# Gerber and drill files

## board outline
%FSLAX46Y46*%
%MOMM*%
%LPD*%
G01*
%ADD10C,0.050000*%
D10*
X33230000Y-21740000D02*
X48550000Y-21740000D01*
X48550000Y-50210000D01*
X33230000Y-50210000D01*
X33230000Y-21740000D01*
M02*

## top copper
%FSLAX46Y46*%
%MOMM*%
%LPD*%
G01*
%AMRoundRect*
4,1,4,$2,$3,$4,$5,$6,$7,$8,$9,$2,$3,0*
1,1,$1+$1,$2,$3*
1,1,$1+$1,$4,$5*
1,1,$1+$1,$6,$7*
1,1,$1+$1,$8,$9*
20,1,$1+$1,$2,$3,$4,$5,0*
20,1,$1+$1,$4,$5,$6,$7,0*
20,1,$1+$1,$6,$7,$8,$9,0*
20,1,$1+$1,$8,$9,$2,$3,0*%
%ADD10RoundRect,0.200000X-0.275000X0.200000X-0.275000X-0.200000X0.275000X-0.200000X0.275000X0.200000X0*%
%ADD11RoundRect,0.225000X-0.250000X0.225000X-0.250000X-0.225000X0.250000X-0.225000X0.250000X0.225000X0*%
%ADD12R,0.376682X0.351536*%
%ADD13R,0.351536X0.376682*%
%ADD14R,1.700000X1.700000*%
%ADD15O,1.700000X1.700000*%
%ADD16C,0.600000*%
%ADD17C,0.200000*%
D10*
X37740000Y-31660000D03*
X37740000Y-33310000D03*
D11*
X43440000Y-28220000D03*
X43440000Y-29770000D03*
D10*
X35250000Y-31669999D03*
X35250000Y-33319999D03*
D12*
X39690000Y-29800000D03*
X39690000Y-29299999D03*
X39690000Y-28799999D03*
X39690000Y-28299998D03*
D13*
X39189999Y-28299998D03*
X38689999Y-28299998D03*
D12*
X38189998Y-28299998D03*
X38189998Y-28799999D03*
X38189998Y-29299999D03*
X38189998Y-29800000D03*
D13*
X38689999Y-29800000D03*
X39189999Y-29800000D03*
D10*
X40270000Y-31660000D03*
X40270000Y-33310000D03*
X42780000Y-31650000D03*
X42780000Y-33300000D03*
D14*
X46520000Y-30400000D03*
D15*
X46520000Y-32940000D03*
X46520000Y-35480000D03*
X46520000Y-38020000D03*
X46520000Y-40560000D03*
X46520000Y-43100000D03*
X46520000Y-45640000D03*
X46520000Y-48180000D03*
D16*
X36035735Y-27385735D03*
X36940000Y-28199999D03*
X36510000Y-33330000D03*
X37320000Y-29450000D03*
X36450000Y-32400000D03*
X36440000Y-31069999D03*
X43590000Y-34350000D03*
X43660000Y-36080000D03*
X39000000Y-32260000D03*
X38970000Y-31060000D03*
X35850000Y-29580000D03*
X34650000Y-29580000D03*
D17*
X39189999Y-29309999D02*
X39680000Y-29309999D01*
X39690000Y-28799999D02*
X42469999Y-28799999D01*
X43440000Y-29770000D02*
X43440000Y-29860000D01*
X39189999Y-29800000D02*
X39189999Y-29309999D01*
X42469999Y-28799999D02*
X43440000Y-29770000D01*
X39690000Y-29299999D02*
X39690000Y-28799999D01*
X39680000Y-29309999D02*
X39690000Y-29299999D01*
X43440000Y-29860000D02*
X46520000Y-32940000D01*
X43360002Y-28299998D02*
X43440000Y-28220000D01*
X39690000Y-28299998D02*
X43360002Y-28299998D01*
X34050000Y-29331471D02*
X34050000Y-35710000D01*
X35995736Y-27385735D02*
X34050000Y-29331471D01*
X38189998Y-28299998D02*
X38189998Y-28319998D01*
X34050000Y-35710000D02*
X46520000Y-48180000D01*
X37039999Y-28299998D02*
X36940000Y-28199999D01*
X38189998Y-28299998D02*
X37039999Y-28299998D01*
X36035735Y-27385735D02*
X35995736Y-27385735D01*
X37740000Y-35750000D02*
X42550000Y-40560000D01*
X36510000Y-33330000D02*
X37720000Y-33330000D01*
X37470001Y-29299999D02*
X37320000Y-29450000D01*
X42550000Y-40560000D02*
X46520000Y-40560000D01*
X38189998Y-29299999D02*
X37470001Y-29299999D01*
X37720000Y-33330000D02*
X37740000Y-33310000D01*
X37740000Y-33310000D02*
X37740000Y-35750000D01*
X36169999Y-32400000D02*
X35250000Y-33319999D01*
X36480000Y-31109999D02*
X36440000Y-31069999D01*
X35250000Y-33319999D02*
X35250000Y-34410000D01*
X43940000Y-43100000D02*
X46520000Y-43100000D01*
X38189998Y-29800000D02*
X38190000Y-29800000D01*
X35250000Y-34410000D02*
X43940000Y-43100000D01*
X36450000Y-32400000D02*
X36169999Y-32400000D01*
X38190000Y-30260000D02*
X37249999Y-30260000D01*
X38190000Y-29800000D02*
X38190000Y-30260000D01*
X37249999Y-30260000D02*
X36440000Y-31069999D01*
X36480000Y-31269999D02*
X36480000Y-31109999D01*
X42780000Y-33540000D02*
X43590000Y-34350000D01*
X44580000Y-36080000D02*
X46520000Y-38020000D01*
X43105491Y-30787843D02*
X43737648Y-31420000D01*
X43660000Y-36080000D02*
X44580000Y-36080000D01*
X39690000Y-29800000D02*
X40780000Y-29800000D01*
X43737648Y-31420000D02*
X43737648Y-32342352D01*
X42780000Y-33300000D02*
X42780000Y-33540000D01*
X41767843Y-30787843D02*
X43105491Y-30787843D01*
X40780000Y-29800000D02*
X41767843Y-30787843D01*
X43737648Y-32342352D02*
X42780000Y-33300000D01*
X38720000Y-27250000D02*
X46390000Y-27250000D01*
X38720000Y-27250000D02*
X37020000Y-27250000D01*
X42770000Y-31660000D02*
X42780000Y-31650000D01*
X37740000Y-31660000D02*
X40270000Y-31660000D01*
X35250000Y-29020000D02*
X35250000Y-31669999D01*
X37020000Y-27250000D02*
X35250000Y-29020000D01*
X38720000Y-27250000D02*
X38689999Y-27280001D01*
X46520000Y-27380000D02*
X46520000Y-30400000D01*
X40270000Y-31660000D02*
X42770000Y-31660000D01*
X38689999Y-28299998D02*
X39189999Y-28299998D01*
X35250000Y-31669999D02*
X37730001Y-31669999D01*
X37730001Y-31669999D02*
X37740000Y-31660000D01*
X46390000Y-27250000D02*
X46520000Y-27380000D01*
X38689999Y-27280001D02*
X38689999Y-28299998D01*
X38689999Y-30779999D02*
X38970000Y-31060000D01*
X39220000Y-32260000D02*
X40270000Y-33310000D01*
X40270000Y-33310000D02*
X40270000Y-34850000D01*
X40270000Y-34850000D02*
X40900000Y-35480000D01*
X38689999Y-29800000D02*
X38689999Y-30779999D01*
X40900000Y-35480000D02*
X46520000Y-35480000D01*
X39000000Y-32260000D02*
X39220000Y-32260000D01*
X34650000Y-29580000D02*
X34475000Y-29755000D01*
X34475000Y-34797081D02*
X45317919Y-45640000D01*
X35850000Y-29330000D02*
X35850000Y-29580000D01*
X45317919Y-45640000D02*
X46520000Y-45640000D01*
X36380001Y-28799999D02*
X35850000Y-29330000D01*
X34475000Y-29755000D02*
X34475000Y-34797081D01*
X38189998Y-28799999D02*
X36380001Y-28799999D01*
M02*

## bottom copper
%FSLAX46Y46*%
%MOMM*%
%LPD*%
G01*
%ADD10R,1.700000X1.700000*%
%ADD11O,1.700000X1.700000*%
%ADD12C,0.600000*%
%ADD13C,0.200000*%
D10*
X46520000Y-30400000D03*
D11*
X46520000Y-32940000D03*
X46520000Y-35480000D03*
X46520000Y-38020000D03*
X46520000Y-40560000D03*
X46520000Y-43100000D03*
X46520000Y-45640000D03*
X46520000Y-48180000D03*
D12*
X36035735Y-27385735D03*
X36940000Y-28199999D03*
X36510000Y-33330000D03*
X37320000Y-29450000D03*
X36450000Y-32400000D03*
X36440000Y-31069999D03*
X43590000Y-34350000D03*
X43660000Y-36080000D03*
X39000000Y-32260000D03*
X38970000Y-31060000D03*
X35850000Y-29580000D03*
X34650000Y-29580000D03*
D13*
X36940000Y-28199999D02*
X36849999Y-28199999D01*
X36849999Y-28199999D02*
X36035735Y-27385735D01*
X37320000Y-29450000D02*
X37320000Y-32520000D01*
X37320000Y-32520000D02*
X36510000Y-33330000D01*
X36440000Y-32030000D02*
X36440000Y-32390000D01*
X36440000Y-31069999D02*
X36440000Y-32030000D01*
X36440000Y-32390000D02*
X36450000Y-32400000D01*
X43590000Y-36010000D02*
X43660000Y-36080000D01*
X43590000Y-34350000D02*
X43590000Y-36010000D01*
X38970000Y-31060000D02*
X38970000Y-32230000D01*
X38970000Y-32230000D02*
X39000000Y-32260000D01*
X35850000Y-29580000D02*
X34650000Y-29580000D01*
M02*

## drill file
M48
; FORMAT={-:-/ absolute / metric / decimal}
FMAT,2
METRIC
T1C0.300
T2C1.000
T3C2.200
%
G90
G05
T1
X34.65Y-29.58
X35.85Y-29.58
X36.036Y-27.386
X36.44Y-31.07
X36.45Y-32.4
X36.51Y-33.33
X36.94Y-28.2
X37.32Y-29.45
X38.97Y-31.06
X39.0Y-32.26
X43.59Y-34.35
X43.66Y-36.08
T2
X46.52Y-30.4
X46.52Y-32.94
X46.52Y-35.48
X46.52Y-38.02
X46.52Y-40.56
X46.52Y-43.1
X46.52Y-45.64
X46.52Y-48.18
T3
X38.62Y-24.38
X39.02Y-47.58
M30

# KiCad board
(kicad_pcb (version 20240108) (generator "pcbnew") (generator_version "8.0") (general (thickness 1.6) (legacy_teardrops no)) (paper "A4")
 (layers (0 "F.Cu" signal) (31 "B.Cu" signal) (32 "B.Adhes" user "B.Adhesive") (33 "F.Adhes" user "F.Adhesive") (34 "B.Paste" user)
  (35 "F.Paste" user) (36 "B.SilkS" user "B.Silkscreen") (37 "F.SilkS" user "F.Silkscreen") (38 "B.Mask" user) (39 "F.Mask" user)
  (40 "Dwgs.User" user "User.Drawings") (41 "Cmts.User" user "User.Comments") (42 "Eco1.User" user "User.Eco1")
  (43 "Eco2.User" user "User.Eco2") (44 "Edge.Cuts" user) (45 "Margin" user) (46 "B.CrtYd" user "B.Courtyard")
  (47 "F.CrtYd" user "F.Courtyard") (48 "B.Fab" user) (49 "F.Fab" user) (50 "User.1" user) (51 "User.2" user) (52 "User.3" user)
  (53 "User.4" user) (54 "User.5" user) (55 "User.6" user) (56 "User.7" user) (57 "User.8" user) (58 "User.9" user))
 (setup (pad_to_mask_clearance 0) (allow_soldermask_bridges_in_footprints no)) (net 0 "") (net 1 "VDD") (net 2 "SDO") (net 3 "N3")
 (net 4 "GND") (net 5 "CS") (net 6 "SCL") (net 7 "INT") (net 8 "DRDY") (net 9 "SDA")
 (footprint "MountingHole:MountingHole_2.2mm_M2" (layer "F.Cu") (at 39.02 47.58)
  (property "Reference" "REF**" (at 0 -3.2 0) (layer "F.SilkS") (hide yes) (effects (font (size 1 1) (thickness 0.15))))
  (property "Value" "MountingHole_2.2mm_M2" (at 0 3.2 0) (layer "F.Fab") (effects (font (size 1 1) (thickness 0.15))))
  (pad "" np_thru_hole circle (at 0 0) (size 2.2 2.2) (drill 2.2) (layers "*.Cu" "*.Mask")))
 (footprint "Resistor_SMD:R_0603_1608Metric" (layer "F.Cu") (at 37.74 32.485 -90)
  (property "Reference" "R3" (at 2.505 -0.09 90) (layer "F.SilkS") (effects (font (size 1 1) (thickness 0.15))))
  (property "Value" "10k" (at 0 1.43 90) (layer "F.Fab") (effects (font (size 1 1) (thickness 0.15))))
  (pad "1" smd roundrect (at -0.825 0 270) (size 0.8 0.95) (layers "F.Cu" "F.Paste" "F.Mask") (roundrect_rratio 0.25) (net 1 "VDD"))
  (pad "2" smd roundrect (at 0.825 0 270) (size 0.8 0.95) (layers "F.Cu" "F.Paste" "F.Mask") (roundrect_rratio 0.25) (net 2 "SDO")))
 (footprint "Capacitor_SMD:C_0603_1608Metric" (layer "F.Cu") (at 43.44 28.995 -90)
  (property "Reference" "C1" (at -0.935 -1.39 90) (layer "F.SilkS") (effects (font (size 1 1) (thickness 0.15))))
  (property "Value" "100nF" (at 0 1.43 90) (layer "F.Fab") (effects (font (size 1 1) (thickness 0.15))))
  (pad "1" smd roundrect (at -0.775 0 270) (size 0.9 0.95) (layers "F.Cu" "F.Paste" "F.Mask") (roundrect_rratio 0.25) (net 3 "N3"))
  (pad "2" smd roundrect (at 0.775 0 270) (size 0.9 0.95) (layers "F.Cu" "F.Paste" "F.Mask") (roundrect_rratio 0.25) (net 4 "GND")))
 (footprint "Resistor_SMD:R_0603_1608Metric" (layer "F.Cu") (at 35.25 32.494999 -90)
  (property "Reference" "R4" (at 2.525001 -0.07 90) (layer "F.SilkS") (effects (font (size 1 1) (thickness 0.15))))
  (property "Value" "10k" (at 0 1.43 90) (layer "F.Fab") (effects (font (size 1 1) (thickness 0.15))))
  (pad "1" smd roundrect (at -0.825 0 270) (size 0.8 0.95) (layers "F.Cu" "F.Paste" "F.Mask") (roundrect_rratio 0.25) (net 1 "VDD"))
  (pad "2" smd roundrect (at 0.825 0 270) (size 0.8 0.95) (layers "F.Cu" "F.Paste" "F.Mask") (roundrect_rratio 0.25) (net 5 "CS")))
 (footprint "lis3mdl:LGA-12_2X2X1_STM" (layer "F.Cu") (at 38.939999 29.049999 180)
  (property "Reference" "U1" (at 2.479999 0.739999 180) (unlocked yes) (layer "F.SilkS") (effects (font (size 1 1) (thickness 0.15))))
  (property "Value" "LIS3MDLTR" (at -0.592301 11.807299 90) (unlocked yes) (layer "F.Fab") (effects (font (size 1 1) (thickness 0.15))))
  (pad "1" smd rect (at -0.750001 -0.750001 180) (size 0.376682 0.351536) (layers "F.Cu" "F.Paste" "F.Mask") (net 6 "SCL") (clearance 0.05))
  (pad "2" smd rect (at -0.750001 -0.25 180) (size 0.376682 0.351536) (layers "F.Cu" "F.Paste" "F.Mask") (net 4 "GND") (clearance 0.05))
  (pad "3" smd rect (at -0.750001 0.25 180) (size 0.376682 0.351536) (layers "F.Cu" "F.Paste" "F.Mask") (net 4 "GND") (clearance 0.05))
  (pad "4" smd rect (at -0.750001 0.750001 180) (size 0.376682 0.351536) (layers "F.Cu" "F.Paste" "F.Mask") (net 3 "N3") (clearance 0.05))
  (pad "5" smd rect (at -0.25 0.750001 270) (size 0.376682 0.351536) (layers "F.Cu" "F.Paste" "F.Mask") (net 1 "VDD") (clearance 0.05))
  (pad "6" smd rect (at 0.25 0.750001 270) (size 0.376682 0.351536) (layers "F.Cu" "F.Paste" "F.Mask") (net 1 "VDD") (clearance 0.05))
  (pad "7" smd rect (at 0.750001 0.750001 180) (size 0.376682 0.351536) (layers "F.Cu" "F.Paste" "F.Mask") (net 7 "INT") (clearance 0.05))
  (pad "8" smd rect (at 0.750001 0.25 180) (size 0.376682 0.351536) (layers "F.Cu" "F.Paste" "F.Mask") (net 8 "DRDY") (clearance 0.05))
  (pad "9" smd rect (at 0.750001 -0.25 180) (size 0.376682 0.351536) (layers "F.Cu" "F.Paste" "F.Mask") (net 2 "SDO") (clearance 0.05))
  (pad "10" smd rect (at 0.750001 -0.750001 180) (size 0.376682 0.351536) (layers "F.Cu" "F.Paste" "F.Mask") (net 5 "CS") (clearance 0.05))
  (pad "11" smd rect (at 0.25 -0.750001 270) (size 0.376682 0.351536) (layers "F.Cu" "F.Paste" "F.Mask") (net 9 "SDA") (clearance 0.05))
  (pad "12" smd rect (at -0.25 -0.750001 270) (size 0.376682 0.351536) (layers "F.Cu" "F.Paste" "F.Mask") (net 4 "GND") (clearance 0.05)))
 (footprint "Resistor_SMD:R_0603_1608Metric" (layer "F.Cu") (at 40.27 32.485 -90)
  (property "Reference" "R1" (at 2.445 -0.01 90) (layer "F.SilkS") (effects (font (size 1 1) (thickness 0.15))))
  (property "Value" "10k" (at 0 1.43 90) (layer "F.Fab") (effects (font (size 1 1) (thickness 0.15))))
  (pad "1" smd roundrect (at -0.825 0 270) (size 0.8 0.95) (layers "F.Cu" "F.Paste" "F.Mask") (roundrect_rratio 0.25) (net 1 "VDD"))
  (pad "2" smd roundrect (at 0.825 0 270) (size 0.8 0.95) (layers "F.Cu" "F.Paste" "F.Mask") (roundrect_rratio 0.25) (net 9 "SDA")))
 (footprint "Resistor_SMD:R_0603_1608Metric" (layer "F.Cu") (at 42.78 32.475 -90)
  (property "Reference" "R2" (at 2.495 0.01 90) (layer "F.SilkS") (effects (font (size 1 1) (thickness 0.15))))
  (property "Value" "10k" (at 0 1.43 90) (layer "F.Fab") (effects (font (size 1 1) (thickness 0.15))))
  (pad "1" smd roundrect (at -0.825 0 270) (size 0.8 0.95) (layers "F.Cu" "F.Paste" "F.Mask") (roundrect_rratio 0.25) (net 1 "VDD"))
  (pad "2" smd roundrect (at 0.825 0 270) (size 0.8 0.95) (layers "F.Cu" "F.Paste" "F.Mask") (roundrect_rratio 0.25) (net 6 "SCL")))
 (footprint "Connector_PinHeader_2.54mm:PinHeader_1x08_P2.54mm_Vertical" (layer "F.Cu") (at 46.52 30.4)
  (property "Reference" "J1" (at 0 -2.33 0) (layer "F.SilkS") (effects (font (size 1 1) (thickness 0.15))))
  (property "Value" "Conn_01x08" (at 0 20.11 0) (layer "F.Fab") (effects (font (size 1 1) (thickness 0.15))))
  (pad "1" thru_hole rect (at 0 0) (size 1.7 1.7) (drill 1) (layers "*.Cu" "*.Mask") (remove_unused_layers no) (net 1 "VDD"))
  (pad "2" thru_hole oval (at 0 2.54) (size 1.7 1.7) (drill 1) (layers "*.Cu" "*.Mask") (remove_unused_layers no) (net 4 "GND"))
  (pad "3" thru_hole oval (at 0 5.08) (size 1.7 1.7) (drill 1) (layers "*.Cu" "*.Mask") (remove_unused_layers no) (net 9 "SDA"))
  (pad "4" thru_hole oval (at 0 7.62) (size 1.7 1.7) (drill 1) (layers "*.Cu" "*.Mask") (remove_unused_layers no) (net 6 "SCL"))
  (pad "5" thru_hole oval (at 0 10.16) (size 1.7 1.7) (drill 1) (layers "*.Cu" "*.Mask") (remove_unused_layers no) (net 2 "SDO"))
  (pad "6" thru_hole oval (at 0 12.7) (size 1.7 1.7) (drill 1) (layers "*.Cu" "*.Mask") (remove_unused_layers no) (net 5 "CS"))
  (pad "7" thru_hole oval (at 0 15.24) (size 1.7 1.7) (drill 1) (layers "*.Cu" "*.Mask") (remove_unused_layers no) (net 8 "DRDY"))
  (pad "8" thru_hole oval (at 0 17.78) (size 1.7 1.7) (drill 1) (layers "*.Cu" "*.Mask") (remove_unused_layers no) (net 7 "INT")))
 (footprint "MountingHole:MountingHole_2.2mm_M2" (layer "F.Cu") (at 38.62 24.38)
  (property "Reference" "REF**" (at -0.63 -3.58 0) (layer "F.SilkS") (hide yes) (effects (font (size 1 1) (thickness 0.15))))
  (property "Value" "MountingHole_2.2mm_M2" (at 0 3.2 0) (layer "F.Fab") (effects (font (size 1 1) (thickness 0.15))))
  (pad "" np_thru_hole circle (at 0 0) (size 2.2 2.2) (drill 2.2) (layers "*.Cu" "*.Mask")))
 (gr_rect (start 33.23 21.74) (end 48.55 50.21) (stroke (width 0.05) (type default)) (fill none) (layer "Edge.Cuts"))
 (segment (start 39.189999 29.309999) (end 39.68 29.309999) (width 0.2) (layer "F.Cu") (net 4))
 (segment (start 39.69 28.799999) (end 42.469999 28.799999) (width 0.2) (layer "F.Cu") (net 4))
 (segment (start 43.44 29.77) (end 43.44 29.86) (width 0.2) (layer "F.Cu") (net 4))
 (segment (start 39.189999 29.8) (end 39.189999 29.309999) (width 0.2) (layer "F.Cu") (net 4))
 (segment (start 42.469999 28.799999) (end 43.44 29.77) (width 0.2) (layer "F.Cu") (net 4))
 (segment (start 39.69 29.299999) (end 39.69 28.799999) (width 0.2) (layer "F.Cu") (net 4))
 (segment (start 39.68 29.309999) (end 39.69 29.299999) (width 0.2) (layer "F.Cu") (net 4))
 (segment (start 43.44 29.86) (end 46.52 32.94) (width 0.2) (layer "F.Cu") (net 4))
 (segment (start 43.360002 28.299998) (end 43.44 28.22) (width 0.2) (layer "F.Cu") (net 3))
 (segment (start 39.69 28.299998) (end 43.360002 28.299998) (width 0.2) (layer "F.Cu") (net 3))
 (segment (start 34.05 29.331471) (end 34.05 35.71) (width 0.2) (layer "F.Cu") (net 7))
 (segment (start 35.995736 27.385735) (end 34.05 29.331471) (width 0.2) (layer "F.Cu") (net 7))
 (segment (start 38.189998 28.299998) (end 38.189998 28.319998) (width 0.2) (layer "F.Cu") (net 7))
 (segment (start 34.05 35.71) (end 46.52 48.18) (width 0.2) (layer "F.Cu") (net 7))
 (segment (start 37.039999 28.299998) (end 36.94 28.199999) (width 0.2) (layer "F.Cu") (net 7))
 (segment (start 38.189998 28.299998) (end 37.039999 28.299998) (width 0.2) (layer "F.Cu") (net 7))
 (segment (start 36.035735 27.385735) (end 35.995736 27.385735) (width 0.2) (layer "F.Cu") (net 7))
 (via (at 36.035735 27.385735) (size 0.6) (drill 0.3) (layers "F.Cu" "B.Cu") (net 7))
 (via (at 36.94 28.199999) (size 0.6) (drill 0.3) (layers "F.Cu" "B.Cu") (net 7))
 (segment (start 36.94 28.199999) (end 36.849999 28.199999) (width 0.2) (layer "B.Cu") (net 7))
 (segment (start 36.849999 28.199999) (end 36.035735 27.385735) (width 0.2) (layer "B.Cu") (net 7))
 (segment (start 37.74 35.75) (end 42.55 40.56) (width 0.2) (layer "F.Cu") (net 2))
 (segment (start 36.51 33.33) (end 37.72 33.33) (width 0.2) (layer "F.Cu") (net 2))
 (segment (start 37.470001 29.299999) (end 37.32 29.45) (width 0.2) (layer "F.Cu") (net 2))
 (segment (start 42.55 40.56) (end 46.52 40.56) (width 0.2) (layer "F.Cu") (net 2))
 (segment (start 38.189998 29.299999) (end 37.470001 29.299999) (width 0.2) (layer "F.Cu") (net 2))
 (segment (start 37.72 33.33) (end 37.74 33.31) (width 0.2) (layer "F.Cu") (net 2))
 (segment (start 37.74 33.31) (end 37.74 35.75) (width 0.2) (layer "F.Cu") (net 2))
 (via (at 36.51 33.33) (size 0.6) (drill 0.3) (layers "F.Cu" "B.Cu") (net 2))
 (via (at 37.32 29.45) (size 0.6) (drill 0.3) (layers "F.Cu" "B.Cu") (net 2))
 (segment (start 37.32 29.45) (end 37.32 32.52) (width 0.2) (layer "B.Cu") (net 2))
 (segment (start 37.32 32.52) (end 36.51 33.33) (width 0.2) (layer "B.Cu") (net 2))
 (segment (start 36.169999 32.4) (end 35.25 33.319999) (width 0.2) (layer "F.Cu") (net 5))
 (segment (start 36.48 31.109999) (end 36.44 31.069999) (width 0.2) (layer "F.Cu") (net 5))
 (segment (start 35.25 33.319999) (end 35.25 34.41) (width 0.2) (layer "F.Cu") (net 5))
 (segment (start 43.94 43.1) (end 46.52 43.1) (width 0.2) (layer "F.Cu") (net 5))
 (segment (start 38.189998 29.8) (end 38.19 29.8) (width 0.2) (layer "F.Cu") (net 5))
 (segment (start 35.25 34.41) (end 43.94 43.1) (width 0.2) (layer "F.Cu") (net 5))
 (segment (start 36.45 32.4) (end 36.169999 32.4) (width 0.2) (layer "F.Cu") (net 5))
 (segment (start 38.19 30.26) (end 37.249999 30.26) (width 0.2) (layer "F.Cu") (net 5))
 (segment (start 38.19 29.8) (end 38.19 30.26) (width 0.2) (layer "F.Cu") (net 5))
 (segment (start 37.249999 30.26) (end 36.44 31.069999) (width 0.2) (layer "F.Cu") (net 5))
 (segment (start 36.48 31.269999) (end 36.48 31.109999) (width 0.2) (layer "F.Cu") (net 5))
 (via (at 36.45 32.4) (size 0.6) (drill 0.3) (layers "F.Cu" "B.Cu") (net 5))
 (via (at 36.44 31.069999) (size 0.6) (drill 0.3) (layers "F.Cu" "B.Cu") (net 5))
 (segment (start 36.44 32.03) (end 36.44 32.39) (width 0.2) (layer "B.Cu") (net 5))
 (segment (start 36.44 31.069999) (end 36.44 32.03) (width 0.2) (layer "B.Cu") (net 5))
 (segment (start 36.44 32.39) (end 36.45 32.4) (width 0.2) (layer "B.Cu") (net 5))
 (segment (start 42.78 33.54) (end 43.59 34.35) (width 0.2) (layer "F.Cu") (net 6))
 (segment (start 44.58 36.08) (end 46.52 38.02) (width 0.2) (layer "F.Cu") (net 6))
 (segment (start 43.105491 30.787843) (end 43.737648 31.42) (width 0.2) (layer "F.Cu") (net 6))
 (segment (start 43.66 36.08) (end 44.58 36.08) (width 0.2) (layer "F.Cu") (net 6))
 (segment (start 39.69 29.8) (end 40.78 29.8) (width 0.2) (layer "F.Cu") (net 6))
 (segment (start 43.737648 31.42) (end 43.737648 32.342352) (width 0.2) (layer "F.Cu") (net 6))
 (segment (start 42.78 33.3) (end 42.78 33.54) (width 0.2) (layer "F.Cu") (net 6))
 (segment (start 41.767843 30.787843) (end 43.105491 30.787843) (width 0.2) (layer "F.Cu") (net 6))
 (segment (start 40.78 29.8) (end 41.767843 30.787843) (width 0.2) (layer "F.Cu") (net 6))
 (segment (start 43.737648 32.342352) (end 42.78 33.3) (width 0.2) (layer "F.Cu") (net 6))
 (via (at 43.59 34.35) (size 0.6) (drill 0.3) (layers "F.Cu" "B.Cu") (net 6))
 (via (at 43.66 36.08) (size 0.6) (drill 0.3) (layers "F.Cu" "B.Cu") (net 6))
 (segment (start 43.59 36.01) (end 43.66 36.08) (width 0.2) (layer "B.Cu") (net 6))
 (segment (start 43.59 34.35) (end 43.59 36.01) (width 0.2) (layer "B.Cu") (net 6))
 (segment (start 38.72 27.25) (end 46.39 27.25) (width 0.2) (layer "F.Cu") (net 1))
 (segment (start 38.72 27.25) (end 37.02 27.25) (width 0.2) (layer "F.Cu") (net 1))
 (segment (start 42.77 31.66) (end 42.78 31.65) (width 0.2) (layer "F.Cu") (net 1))
 (segment (start 37.74 31.66) (end 40.27 31.66) (width 0.2) (layer "F.Cu") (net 1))
 (segment (start 35.25 29.02) (end 35.25 31.669999) (width 0.2) (layer "F.Cu") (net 1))
 (segment (start 37.02 27.25) (end 35.25 29.02) (width 0.2) (layer "F.Cu") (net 1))
 (segment (start 38.72 27.25) (end 38.689999 27.280001) (width 0.2) (layer "F.Cu") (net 1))
 (segment (start 46.52 27.38) (end 46.52 30.4) (width 0.2) (layer "F.Cu") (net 1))
 (segment (start 40.27 31.66) (end 42.77 31.66) (width 0.2) (layer "F.Cu") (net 1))
 (segment (start 38.689999 28.299998) (end 39.189999 28.299998) (width 0.2) (layer "F.Cu") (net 1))
 (segment (start 35.25 31.669999) (end 37.730001 31.669999) (width 0.2) (layer "F.Cu") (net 1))
 (segment (start 37.730001 31.669999) (end 37.74 31.66) (width 0.2) (layer "F.Cu") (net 1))
 (segment (start 46.39 27.25) (end 46.52 27.38) (width 0.2) (layer "F.Cu") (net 1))
 (segment (start 38.689999 27.280001) (end 38.689999 28.299998) (width 0.2) (layer "F.Cu") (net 1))
 (segment (start 38.689999 30.779999) (end 38.97 31.06) (width 0.2) (layer "F.Cu") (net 9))
 (segment (start 39.22 32.26) (end 40.27 33.31) (width 0.2) (layer "F.Cu") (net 9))
 (segment (start 40.27 33.31) (end 40.27 34.85) (width 0.2) (layer "F.Cu") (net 9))
 (segment (start 40.27 34.85) (end 40.9 35.48) (width 0.2) (layer "F.Cu") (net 9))
 (segment (start 38.689999 29.8) (end 38.689999 30.779999) (width 0.2) (layer "F.Cu") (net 9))
 (segment (start 40.9 35.48) (end 46.52 35.48) (width 0.2) (layer "F.Cu") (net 9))
 (segment (start 39 32.26) (end 39.22 32.26) (width 0.2) (layer "F.Cu") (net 9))
 (via (at 39 32.26) (size 0.6) (drill 0.3) (layers "F.Cu" "B.Cu") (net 9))
 (via (at 38.97 31.06) (size 0.6) (drill 0.3) (layers "F.Cu" "B.Cu") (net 9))
 (segment (start 38.97 31.06) (end 38.97 32.23) (width 0.2) (layer "B.Cu") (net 9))
 (segment (start 38.97 32.23) (end 39 32.26) (width 0.2) (layer "B.Cu") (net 9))
 (segment (start 34.65 29.58) (end 34.475 29.755) (width 0.2) (layer "F.Cu") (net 8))
 (segment (start 34.475 34.797081) (end 45.317919 45.64) (width 0.2) (layer "F.Cu") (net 8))
 (segment (start 35.85 29.33) (end 35.85 29.58) (width 0.2) (layer "F.Cu") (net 8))
 (segment (start 45.317919 45.64) (end 46.52 45.64) (width 0.2) (layer "F.Cu") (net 8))
 (segment (start 36.380001 28.799999) (end 35.85 29.33) (width 0.2) (layer "F.Cu") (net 8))
 (segment (start 34.475 29.755) (end 34.475 34.797081) (width 0.2) (layer "F.Cu") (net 8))
 (segment (start 38.189998 28.799999) (end 36.380001 28.799999) (width 0.2) (layer "F.Cu") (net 8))
 (via (at 35.85 29.58) (size 0.6) (drill 0.3) (layers "F.Cu" "B.Cu") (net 8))
 (via (at 34.65 29.58) (size 0.6) (drill 0.3) (layers "F.Cu" "B.Cu") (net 8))
 (segment (start 35.85 29.58) (end 34.65 29.58) (width 0.2) (layer "B.Cu") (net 8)))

